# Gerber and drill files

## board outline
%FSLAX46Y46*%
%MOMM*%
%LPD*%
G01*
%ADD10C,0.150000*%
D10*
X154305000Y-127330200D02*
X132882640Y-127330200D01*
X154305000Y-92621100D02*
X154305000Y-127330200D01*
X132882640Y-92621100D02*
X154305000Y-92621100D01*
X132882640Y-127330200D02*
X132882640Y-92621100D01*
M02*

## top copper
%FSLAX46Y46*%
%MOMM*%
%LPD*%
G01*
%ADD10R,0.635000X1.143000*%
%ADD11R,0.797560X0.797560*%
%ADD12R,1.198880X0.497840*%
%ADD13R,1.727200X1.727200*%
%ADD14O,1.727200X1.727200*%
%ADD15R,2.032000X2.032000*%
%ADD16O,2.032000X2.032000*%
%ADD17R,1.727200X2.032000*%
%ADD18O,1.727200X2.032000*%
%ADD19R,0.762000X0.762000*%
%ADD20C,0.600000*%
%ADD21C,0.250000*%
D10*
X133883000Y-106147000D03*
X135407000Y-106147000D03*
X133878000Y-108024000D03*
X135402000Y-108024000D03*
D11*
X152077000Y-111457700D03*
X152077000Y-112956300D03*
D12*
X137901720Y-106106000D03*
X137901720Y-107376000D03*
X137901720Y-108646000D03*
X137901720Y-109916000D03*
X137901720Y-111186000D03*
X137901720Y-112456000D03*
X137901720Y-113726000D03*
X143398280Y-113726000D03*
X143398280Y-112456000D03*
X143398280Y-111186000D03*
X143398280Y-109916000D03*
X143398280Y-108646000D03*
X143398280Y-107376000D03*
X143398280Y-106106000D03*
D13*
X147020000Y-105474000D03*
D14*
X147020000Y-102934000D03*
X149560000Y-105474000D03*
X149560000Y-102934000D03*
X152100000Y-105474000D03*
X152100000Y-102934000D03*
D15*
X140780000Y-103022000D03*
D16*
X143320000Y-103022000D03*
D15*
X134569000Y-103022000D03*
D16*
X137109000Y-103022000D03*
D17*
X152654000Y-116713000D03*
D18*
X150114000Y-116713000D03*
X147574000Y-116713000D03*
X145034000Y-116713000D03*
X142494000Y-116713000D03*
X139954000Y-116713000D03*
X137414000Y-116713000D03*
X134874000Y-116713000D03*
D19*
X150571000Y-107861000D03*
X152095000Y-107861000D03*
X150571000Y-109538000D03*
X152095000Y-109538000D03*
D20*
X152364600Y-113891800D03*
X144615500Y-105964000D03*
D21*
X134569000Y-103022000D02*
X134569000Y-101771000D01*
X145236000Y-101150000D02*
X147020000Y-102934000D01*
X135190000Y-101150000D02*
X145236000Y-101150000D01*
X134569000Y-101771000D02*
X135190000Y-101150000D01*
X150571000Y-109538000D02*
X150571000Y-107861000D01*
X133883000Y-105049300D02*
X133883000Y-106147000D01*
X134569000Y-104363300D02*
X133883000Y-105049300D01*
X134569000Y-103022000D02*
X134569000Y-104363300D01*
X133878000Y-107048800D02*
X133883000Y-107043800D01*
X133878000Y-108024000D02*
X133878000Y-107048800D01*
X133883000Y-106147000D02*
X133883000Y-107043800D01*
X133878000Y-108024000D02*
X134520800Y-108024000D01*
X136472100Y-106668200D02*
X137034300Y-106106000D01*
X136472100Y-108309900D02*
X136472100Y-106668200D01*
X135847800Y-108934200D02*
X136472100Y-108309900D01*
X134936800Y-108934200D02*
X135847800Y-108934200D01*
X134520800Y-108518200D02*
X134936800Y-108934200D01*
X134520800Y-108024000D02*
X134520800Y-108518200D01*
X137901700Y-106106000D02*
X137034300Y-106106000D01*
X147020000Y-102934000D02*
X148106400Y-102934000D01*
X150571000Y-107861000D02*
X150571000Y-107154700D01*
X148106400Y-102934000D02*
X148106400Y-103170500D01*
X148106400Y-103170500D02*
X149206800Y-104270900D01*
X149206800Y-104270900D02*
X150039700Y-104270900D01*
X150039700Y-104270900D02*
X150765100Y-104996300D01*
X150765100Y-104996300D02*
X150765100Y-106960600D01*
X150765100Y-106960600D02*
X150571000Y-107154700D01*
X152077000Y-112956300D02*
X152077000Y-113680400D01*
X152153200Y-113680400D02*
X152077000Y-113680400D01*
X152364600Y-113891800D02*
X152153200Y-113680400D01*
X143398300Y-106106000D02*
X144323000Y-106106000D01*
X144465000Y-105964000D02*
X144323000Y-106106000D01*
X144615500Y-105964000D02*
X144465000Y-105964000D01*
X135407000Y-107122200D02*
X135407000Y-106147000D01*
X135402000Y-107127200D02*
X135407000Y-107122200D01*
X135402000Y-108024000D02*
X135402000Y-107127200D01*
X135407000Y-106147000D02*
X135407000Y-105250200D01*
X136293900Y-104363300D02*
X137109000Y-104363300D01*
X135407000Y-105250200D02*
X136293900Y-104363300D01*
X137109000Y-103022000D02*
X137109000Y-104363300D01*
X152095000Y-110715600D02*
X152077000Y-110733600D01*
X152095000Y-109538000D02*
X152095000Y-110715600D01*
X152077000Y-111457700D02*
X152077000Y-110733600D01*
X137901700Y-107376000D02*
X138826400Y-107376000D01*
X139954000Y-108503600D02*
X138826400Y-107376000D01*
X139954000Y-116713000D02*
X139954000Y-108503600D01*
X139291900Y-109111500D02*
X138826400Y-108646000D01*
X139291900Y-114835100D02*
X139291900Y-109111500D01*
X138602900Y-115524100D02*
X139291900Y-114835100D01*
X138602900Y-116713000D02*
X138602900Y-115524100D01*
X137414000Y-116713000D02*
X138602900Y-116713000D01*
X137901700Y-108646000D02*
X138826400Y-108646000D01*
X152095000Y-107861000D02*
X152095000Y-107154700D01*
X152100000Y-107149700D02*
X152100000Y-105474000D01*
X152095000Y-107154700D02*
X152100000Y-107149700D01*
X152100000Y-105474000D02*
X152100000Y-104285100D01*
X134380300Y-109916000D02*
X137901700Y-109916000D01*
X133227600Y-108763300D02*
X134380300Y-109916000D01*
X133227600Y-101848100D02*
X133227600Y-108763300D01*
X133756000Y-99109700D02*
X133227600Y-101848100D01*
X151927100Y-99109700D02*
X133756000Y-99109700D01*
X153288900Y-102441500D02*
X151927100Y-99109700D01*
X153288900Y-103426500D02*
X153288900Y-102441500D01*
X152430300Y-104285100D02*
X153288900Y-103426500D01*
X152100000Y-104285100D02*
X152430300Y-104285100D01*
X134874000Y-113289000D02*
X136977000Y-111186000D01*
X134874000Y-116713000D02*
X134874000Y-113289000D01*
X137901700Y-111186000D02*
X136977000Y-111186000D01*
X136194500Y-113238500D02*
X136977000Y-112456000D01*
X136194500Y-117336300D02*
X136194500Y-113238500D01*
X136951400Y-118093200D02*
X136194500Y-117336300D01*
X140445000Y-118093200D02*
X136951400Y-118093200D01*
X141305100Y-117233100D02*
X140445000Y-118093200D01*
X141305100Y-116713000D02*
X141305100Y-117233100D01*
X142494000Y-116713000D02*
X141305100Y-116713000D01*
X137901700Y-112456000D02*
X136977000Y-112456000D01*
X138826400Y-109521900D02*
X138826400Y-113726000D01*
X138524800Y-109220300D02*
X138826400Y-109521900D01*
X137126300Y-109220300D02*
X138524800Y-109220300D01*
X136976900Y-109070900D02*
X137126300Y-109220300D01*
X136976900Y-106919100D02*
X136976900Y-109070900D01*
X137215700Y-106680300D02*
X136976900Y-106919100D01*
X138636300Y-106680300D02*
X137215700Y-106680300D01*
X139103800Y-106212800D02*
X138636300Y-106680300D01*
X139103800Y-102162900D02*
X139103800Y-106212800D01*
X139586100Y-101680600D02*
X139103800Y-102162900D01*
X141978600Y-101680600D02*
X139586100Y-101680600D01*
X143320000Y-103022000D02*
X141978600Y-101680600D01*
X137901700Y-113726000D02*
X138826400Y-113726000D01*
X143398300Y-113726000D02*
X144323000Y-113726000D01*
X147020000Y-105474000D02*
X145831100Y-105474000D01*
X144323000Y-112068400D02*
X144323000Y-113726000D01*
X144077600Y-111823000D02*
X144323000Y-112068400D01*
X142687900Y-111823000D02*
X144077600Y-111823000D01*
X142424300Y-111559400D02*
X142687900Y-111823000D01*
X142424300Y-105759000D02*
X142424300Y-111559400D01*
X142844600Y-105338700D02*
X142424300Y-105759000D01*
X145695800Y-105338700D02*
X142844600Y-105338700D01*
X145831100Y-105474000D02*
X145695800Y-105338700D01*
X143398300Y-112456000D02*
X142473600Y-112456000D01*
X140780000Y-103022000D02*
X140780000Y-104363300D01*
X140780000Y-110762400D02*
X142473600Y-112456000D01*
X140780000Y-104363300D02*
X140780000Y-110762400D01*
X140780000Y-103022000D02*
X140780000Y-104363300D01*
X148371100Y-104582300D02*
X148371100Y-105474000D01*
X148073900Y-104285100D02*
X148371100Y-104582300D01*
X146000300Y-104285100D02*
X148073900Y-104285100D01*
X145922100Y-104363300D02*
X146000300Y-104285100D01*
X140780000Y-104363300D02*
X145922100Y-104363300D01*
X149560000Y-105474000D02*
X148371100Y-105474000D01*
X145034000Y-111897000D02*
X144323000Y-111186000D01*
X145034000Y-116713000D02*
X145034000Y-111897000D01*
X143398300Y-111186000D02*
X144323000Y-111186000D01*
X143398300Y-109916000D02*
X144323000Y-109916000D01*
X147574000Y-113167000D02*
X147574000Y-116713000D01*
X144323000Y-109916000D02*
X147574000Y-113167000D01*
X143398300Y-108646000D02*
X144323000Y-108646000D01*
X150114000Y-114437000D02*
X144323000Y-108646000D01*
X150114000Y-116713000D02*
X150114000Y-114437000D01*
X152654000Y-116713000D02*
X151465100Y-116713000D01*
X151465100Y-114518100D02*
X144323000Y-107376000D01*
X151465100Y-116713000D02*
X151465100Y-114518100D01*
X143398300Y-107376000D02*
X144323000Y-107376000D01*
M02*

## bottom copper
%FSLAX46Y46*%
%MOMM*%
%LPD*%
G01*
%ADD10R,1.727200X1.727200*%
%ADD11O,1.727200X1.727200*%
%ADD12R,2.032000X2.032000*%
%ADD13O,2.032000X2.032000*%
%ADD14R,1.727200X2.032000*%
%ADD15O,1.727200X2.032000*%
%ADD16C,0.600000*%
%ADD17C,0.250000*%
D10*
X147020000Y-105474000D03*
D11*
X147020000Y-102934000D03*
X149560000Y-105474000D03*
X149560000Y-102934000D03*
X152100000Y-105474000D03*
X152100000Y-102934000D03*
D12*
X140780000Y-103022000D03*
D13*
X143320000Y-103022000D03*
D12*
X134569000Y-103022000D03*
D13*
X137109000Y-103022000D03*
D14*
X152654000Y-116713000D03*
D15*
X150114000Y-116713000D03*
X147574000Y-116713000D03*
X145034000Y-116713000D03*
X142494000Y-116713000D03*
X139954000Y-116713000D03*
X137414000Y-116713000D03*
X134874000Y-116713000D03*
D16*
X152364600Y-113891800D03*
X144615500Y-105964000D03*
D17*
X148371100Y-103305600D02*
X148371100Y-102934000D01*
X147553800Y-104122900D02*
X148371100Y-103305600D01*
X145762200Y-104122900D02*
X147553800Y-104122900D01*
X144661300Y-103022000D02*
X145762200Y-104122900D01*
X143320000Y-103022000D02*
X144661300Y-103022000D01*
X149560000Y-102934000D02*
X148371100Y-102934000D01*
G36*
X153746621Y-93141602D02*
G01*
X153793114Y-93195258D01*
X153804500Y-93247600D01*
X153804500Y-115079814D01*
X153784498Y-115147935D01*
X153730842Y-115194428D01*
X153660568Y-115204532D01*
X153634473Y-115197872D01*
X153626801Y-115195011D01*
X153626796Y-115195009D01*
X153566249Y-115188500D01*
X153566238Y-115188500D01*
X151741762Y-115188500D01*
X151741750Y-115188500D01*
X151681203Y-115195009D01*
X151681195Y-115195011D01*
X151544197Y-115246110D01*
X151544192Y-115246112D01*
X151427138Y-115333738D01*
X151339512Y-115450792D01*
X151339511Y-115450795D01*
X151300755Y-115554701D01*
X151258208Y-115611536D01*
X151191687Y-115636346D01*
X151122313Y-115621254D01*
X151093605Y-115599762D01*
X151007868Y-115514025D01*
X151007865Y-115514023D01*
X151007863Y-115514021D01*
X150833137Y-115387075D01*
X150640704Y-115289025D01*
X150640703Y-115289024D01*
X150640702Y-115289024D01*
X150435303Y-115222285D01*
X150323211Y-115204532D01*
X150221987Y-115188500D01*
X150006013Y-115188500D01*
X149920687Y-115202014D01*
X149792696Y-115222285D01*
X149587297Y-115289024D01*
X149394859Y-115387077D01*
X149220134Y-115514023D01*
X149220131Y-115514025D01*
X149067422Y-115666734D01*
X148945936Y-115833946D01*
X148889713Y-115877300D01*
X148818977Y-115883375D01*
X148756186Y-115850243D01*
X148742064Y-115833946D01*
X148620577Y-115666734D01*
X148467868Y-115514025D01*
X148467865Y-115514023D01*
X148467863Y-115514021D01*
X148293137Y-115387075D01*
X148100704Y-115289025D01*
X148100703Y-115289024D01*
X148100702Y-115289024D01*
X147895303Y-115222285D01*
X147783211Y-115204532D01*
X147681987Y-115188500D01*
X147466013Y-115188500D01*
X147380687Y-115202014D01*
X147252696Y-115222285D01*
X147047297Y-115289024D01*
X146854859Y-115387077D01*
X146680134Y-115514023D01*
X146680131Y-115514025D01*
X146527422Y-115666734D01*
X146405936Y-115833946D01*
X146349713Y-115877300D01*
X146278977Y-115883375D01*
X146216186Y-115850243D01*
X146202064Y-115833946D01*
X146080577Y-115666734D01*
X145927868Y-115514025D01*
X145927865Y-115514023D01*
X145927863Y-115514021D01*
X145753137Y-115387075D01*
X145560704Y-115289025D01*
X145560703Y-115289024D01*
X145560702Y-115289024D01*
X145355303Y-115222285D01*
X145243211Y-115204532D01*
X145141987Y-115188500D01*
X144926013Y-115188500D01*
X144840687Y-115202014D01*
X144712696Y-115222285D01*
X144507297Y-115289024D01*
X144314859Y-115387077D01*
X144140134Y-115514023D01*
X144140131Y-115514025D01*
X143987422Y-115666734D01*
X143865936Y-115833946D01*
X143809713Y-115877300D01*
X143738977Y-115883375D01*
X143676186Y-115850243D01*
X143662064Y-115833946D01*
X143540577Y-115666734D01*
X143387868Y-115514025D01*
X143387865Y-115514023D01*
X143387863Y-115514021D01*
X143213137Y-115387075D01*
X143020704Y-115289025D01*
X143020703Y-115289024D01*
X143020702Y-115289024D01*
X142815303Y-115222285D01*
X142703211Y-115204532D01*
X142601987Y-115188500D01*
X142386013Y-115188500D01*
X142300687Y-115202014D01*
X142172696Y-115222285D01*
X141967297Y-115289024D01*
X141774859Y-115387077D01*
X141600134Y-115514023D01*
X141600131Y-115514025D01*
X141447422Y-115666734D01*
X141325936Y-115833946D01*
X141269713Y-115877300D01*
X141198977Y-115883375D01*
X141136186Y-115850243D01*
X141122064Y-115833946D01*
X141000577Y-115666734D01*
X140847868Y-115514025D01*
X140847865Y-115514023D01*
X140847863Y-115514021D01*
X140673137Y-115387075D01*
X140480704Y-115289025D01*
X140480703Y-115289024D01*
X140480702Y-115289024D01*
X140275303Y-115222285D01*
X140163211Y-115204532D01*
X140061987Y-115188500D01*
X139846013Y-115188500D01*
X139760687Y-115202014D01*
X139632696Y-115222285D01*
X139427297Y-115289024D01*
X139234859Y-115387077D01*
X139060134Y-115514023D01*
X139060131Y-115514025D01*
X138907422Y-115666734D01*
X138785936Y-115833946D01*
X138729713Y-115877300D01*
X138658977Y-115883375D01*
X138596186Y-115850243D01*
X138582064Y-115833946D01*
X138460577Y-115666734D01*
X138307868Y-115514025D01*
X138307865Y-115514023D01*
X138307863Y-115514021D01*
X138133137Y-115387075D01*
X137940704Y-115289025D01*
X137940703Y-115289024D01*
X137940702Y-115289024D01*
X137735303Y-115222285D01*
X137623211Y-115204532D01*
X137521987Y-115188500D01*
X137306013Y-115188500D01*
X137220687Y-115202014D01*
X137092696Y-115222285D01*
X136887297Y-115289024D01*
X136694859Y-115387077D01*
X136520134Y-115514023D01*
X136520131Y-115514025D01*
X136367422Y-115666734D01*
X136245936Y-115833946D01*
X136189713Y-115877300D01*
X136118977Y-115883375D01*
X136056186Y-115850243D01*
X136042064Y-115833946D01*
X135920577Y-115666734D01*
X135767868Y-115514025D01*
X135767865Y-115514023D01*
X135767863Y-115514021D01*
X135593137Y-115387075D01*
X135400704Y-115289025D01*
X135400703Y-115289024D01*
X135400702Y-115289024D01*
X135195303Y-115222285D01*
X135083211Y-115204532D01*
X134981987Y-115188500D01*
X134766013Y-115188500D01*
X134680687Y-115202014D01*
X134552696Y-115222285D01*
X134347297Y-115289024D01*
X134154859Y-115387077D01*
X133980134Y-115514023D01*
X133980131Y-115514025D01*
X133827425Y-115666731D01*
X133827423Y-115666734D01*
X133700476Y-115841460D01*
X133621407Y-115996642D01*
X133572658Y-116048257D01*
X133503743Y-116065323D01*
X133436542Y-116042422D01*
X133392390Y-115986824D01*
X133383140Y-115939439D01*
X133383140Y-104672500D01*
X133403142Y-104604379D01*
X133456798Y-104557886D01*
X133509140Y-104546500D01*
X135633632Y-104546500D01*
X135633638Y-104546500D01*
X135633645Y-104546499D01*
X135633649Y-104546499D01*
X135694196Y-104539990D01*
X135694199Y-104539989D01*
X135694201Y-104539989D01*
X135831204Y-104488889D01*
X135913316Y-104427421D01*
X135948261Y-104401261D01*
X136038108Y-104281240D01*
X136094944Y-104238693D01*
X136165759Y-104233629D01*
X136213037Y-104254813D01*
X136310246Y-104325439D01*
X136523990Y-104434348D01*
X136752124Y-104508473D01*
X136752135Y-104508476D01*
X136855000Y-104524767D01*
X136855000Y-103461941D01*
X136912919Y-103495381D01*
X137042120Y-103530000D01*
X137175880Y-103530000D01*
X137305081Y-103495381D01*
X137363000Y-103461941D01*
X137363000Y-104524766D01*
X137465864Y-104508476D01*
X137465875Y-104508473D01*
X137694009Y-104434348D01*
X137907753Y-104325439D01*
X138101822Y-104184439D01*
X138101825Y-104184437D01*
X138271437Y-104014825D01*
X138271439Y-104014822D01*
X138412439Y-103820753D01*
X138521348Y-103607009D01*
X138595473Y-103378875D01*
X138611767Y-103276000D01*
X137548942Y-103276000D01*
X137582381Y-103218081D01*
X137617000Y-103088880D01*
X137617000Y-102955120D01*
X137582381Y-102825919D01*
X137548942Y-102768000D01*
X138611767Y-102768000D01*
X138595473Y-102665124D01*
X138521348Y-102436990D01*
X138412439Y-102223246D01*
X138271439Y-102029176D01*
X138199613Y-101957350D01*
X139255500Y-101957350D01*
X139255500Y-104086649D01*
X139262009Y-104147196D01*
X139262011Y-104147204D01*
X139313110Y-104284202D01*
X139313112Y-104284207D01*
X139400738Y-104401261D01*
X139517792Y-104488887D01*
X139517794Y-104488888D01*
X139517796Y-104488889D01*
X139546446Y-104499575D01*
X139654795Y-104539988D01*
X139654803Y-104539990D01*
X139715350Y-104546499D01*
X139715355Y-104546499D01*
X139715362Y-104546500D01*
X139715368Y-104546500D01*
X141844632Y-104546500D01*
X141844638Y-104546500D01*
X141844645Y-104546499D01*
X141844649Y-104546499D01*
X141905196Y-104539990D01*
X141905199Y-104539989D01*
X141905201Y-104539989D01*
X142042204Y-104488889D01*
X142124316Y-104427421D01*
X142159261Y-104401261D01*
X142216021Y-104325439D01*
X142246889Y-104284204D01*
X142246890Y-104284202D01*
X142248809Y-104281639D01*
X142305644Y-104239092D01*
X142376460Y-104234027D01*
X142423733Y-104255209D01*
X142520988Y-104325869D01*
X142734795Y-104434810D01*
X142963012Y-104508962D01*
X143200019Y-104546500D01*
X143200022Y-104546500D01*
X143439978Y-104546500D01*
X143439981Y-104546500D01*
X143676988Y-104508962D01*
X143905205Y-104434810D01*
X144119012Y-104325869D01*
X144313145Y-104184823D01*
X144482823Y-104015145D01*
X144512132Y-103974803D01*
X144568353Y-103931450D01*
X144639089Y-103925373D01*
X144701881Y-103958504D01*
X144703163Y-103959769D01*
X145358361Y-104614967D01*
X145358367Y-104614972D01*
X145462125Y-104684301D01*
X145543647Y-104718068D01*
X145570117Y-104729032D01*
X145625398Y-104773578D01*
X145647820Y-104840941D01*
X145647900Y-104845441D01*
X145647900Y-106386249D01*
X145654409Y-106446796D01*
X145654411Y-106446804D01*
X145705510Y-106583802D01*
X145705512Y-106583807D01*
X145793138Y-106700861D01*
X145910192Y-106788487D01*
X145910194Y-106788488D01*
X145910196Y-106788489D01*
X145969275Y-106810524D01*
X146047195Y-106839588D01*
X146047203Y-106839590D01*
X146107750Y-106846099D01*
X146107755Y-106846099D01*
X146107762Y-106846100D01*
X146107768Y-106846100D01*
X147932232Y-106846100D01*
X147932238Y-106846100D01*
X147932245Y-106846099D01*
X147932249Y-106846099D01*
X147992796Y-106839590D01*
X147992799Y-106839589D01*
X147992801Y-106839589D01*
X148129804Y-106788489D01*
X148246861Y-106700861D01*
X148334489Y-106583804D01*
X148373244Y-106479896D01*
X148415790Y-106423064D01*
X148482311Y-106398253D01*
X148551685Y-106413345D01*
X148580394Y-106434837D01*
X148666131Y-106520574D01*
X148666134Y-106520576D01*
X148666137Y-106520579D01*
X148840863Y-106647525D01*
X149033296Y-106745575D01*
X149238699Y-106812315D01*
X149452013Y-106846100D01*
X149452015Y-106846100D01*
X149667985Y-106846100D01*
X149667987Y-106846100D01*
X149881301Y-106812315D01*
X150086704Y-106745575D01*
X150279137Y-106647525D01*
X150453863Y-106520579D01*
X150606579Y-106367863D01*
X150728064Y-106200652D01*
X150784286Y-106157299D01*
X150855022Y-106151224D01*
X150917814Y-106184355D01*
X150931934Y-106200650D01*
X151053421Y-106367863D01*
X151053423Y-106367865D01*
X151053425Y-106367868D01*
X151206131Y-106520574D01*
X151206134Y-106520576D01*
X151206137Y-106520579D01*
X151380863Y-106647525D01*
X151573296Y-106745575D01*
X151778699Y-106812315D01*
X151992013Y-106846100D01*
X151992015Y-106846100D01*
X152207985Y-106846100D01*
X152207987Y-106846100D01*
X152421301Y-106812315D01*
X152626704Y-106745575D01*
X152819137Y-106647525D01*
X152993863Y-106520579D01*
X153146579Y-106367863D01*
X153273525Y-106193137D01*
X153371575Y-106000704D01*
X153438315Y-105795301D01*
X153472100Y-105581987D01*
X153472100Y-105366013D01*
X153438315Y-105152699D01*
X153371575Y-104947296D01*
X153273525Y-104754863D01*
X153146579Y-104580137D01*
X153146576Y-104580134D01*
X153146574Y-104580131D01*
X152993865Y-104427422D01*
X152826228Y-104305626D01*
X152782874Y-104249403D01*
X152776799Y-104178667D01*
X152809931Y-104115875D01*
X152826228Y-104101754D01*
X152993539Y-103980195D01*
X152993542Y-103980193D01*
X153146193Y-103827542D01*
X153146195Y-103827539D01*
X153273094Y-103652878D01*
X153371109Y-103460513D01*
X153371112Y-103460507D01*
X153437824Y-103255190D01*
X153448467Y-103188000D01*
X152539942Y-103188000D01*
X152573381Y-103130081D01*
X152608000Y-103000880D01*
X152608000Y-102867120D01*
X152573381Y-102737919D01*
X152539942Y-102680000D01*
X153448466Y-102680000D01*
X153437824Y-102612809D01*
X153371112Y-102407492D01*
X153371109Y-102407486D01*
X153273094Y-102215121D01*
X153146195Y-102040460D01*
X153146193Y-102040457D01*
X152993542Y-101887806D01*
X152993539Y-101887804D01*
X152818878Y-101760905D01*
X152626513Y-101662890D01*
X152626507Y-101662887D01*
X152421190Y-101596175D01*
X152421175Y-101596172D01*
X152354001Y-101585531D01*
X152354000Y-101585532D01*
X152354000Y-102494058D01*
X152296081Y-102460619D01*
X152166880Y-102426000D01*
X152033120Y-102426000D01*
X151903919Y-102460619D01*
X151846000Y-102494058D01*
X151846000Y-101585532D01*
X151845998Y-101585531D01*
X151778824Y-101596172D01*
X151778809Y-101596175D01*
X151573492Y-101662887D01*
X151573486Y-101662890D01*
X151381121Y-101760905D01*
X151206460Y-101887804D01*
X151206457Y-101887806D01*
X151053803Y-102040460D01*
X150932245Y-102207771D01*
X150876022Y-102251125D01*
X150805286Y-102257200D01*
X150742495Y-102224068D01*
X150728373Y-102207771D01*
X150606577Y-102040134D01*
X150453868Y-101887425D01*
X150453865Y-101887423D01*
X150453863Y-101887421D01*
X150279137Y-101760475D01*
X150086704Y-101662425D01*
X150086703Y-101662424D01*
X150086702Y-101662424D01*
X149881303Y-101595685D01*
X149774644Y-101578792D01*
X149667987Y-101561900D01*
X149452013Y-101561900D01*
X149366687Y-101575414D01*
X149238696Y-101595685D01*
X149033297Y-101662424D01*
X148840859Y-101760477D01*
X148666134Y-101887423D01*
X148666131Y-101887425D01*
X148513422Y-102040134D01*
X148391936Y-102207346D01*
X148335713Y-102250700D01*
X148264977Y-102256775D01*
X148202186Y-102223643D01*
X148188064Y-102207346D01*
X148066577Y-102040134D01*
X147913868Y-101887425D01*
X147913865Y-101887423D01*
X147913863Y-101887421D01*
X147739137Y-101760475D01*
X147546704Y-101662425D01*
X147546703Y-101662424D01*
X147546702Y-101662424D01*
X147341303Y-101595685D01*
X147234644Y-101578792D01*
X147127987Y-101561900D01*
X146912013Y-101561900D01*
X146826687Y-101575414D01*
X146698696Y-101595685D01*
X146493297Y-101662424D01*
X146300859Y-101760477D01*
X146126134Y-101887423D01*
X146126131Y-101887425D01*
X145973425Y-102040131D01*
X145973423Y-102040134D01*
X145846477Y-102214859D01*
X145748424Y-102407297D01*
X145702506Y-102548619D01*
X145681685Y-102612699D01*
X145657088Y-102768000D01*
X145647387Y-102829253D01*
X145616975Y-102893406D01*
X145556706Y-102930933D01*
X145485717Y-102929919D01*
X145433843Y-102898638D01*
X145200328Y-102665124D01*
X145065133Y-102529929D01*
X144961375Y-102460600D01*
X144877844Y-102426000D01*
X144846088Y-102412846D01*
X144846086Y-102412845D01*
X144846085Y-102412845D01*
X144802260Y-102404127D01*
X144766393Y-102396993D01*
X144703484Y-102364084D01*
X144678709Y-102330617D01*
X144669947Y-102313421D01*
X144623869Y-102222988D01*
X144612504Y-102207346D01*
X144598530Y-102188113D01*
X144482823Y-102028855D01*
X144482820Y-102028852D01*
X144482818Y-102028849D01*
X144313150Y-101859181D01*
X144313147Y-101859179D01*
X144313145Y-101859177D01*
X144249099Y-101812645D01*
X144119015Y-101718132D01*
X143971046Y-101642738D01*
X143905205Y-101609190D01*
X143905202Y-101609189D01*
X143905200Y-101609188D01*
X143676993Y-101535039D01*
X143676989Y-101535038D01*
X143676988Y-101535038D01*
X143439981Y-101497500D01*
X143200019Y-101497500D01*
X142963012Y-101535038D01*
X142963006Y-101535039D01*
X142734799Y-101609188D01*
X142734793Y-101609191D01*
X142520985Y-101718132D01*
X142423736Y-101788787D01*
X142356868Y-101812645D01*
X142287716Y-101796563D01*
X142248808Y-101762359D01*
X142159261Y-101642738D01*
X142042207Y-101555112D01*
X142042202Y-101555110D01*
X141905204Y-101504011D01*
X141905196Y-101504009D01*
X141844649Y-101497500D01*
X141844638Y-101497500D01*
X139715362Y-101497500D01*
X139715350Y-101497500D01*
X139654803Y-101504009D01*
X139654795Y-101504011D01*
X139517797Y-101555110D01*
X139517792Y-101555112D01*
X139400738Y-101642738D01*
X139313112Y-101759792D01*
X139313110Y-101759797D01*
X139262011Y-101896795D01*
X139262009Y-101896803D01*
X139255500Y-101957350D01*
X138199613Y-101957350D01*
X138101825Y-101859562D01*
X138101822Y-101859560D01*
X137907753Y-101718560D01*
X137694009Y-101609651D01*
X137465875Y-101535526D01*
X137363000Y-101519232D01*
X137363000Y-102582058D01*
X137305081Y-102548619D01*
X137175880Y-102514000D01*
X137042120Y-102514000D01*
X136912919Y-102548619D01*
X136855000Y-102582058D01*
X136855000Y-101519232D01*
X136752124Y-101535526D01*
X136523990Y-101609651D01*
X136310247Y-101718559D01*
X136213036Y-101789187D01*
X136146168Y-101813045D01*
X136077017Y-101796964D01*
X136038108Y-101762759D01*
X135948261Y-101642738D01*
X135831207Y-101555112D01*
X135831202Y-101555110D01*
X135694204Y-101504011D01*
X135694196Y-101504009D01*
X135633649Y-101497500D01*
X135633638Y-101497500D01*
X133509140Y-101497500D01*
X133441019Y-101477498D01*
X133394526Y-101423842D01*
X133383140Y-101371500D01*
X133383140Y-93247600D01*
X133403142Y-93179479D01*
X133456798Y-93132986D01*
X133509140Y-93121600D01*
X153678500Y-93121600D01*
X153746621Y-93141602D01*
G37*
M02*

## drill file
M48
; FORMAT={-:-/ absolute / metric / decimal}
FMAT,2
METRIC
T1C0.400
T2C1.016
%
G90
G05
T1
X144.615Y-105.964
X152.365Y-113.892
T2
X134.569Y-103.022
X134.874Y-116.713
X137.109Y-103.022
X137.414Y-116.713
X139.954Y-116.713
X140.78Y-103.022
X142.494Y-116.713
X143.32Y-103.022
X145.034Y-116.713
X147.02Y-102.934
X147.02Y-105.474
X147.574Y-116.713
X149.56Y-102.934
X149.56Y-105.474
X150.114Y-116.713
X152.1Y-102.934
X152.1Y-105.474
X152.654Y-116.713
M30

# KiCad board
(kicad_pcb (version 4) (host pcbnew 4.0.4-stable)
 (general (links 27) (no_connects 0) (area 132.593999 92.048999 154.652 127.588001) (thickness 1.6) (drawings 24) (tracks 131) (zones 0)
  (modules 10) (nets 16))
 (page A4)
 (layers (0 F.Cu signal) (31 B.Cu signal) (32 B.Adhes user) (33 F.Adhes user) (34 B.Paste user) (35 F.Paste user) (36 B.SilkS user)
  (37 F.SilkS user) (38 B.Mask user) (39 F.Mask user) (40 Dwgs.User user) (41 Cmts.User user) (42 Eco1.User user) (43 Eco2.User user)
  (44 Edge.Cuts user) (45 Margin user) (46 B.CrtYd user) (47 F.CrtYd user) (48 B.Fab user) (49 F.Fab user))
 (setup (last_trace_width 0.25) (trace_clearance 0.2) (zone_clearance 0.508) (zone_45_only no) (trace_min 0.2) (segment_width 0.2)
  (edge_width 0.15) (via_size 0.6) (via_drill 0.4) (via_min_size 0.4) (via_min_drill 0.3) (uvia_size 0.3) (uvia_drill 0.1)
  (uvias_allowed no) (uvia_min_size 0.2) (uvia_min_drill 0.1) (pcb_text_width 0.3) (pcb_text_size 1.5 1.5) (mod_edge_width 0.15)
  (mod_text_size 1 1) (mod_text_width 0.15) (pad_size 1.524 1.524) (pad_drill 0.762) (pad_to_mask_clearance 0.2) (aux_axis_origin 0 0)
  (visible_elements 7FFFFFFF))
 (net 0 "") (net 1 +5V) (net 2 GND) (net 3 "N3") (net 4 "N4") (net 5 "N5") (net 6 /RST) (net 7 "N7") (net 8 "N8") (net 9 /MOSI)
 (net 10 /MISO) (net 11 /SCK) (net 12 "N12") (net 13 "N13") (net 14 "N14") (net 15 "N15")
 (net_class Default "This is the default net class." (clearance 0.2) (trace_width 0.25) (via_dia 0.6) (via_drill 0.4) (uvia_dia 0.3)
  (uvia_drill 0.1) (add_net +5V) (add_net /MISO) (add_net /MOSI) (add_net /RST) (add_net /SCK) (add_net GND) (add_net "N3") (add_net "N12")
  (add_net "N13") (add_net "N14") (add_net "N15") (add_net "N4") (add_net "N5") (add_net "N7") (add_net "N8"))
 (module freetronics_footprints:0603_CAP (layer F.Cu) (at 134.645 106.147)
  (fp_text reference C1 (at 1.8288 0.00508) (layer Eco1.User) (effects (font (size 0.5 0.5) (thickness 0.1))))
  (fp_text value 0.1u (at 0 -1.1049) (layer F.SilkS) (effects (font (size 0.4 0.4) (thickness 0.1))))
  (pad 1 smd rect (at -0.762 0) (size 0.635 1.143) (layers F.Cu F.Paste F.Mask) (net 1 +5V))
  (pad 2 smd rect (at 0.762 0) (size 0.635 1.143) (layers F.Cu F.Paste F.Mask) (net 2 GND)))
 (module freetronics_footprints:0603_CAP (layer F.Cu) (at 134.64 108.024)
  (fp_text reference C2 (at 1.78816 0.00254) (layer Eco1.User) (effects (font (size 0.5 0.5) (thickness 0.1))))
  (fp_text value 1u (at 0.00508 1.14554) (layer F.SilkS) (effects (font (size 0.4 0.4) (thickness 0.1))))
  (pad 1 smd rect (at -0.762 0) (size 0.635 1.143) (layers F.Cu F.Paste F.Mask) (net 1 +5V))
  (pad 2 smd rect (at 0.762 0) (size 0.635 1.143) (layers F.Cu F.Paste F.Mask) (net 2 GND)))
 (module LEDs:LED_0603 (layer F.Cu) (at 152.077 112.207 90)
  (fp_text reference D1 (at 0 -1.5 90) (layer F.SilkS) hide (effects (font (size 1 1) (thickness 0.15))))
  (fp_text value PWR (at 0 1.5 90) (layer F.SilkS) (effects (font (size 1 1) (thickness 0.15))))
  (pad 2 smd rect (at 0.7493 0 270) (size 0.79756 0.79756) (layers F.Cu F.Paste F.Mask) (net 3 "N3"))
  (pad 1 smd rect (at -0.7493 0 270) (size 0.79756 0.79756) (layers F.Cu F.Paste F.Mask) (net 2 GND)))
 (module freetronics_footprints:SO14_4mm (layer F.Cu) (at 140.65 109.916 270)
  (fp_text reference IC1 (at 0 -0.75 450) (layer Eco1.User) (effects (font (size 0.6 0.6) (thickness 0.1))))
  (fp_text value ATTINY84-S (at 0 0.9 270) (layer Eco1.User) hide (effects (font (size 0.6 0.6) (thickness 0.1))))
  (pad 1 smd rect (at -3.81 2.74828 90) (size 0.49784 1.19888) (layers F.Cu F.Paste F.Mask) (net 1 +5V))
  (pad 2 smd rect (at -2.54 2.74828 90) (size 0.49784 1.19888) (layers F.Cu F.Paste F.Mask) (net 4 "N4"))
  (pad 3 smd rect (at -1.27 2.74828 90) (size 0.49784 1.19888) (layers F.Cu F.Paste F.Mask) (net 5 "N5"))
  (pad 4 smd rect (at 0 2.74828 90) (size 0.49784 1.19888) (layers F.Cu F.Paste F.Mask) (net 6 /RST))
  (pad 5 smd rect (at 1.27 2.74828 90) (size 0.49784 1.19888) (layers F.Cu F.Paste F.Mask) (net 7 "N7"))
  (pad 6 smd rect (at 2.54 2.74828 90) (size 0.49784 1.19888) (layers F.Cu F.Paste F.Mask) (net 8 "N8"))
  (pad 7 smd rect (at 3.81 2.74828 90) (size 0.49784 1.19888) (layers F.Cu F.Paste F.Mask) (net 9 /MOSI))
  (pad 8 smd rect (at 3.81 -2.74828 270) (size 0.49784 1.19888) (layers F.Cu F.Paste F.Mask) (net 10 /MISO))
  (pad 9 smd rect (at 2.54 -2.74828 270) (size 0.49784 1.19888) (layers F.Cu F.Paste F.Mask) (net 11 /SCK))
  (pad 10 smd rect (at 1.27 -2.74828 270) (size 0.49784 1.19888) (layers F.Cu F.Paste F.Mask) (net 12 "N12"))
  (pad 11 smd rect (at 0 -2.74828 270) (size 0.49784 1.19888) (layers F.Cu F.Paste F.Mask) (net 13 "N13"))
  (pad 12 smd rect (at -1.27 -2.74828 270) (size 0.49784 1.19888) (layers F.Cu F.Paste F.Mask) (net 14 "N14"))
  (pad 13 smd rect (at -2.54 -2.74828 270) (size 0.49784 1.19888) (layers F.Cu F.Paste F.Mask) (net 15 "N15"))
  (pad 14 smd rect (at -3.81 -2.74828 270) (size 0.49784 1.19888) (layers F.Cu F.Paste F.Mask) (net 2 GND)))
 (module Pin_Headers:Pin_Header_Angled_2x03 (layer F.Cu) (at 147.02 105.474 90)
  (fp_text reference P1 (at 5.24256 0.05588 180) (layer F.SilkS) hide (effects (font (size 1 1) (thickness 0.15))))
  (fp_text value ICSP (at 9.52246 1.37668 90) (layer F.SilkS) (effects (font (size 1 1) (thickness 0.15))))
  (pad 1 thru_hole rect (at 0 0 90) (size 1.7272 1.7272) (drill 1.016) (layers *.Cu *.Mask F.SilkS) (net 10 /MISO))
  (pad 2 thru_hole oval (at 2.54 0 90) (size 1.7272 1.7272) (drill 1.016) (layers *.Cu *.Mask F.SilkS) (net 1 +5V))
  (pad 3 thru_hole oval (at 0 2.54 90) (size 1.7272 1.7272) (drill 1.016) (layers *.Cu *.Mask F.SilkS) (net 11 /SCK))
  (pad 4 thru_hole oval (at 2.54 2.54 90) (size 1.7272 1.7272) (drill 1.016) (layers *.Cu *.Mask F.SilkS) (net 9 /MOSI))
  (pad 5 thru_hole oval (at 0 5.08 90) (size 1.7272 1.7272) (drill 1.016) (layers *.Cu *.Mask F.SilkS) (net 6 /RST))
  (pad 6 thru_hole oval (at 2.54 5.08 90) (size 1.7272 1.7272) (drill 1.016) (layers *.Cu *.Mask F.SilkS) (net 2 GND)))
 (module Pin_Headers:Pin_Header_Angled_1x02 (layer F.Cu) (at 140.78 103.022 90)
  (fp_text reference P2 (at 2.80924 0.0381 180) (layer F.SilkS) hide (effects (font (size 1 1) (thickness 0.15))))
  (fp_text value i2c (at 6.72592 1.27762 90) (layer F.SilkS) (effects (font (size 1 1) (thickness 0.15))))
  (pad 1 thru_hole rect (at 0 0 90) (size 2.032 2.032) (drill 1.016) (layers *.Cu *.Mask F.SilkS) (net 11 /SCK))
  (pad 2 thru_hole oval (at 0 2.54 90) (size 2.032 2.032) (drill 1.016) (layers *.Cu *.Mask F.SilkS) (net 9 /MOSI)))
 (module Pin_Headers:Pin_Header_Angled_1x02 (layer F.Cu) (at 134.569 103.022 90)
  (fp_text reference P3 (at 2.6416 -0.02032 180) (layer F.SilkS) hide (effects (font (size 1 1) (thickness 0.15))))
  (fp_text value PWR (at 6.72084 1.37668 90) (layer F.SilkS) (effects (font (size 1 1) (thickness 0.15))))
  (pad 1 thru_hole rect (at 0 0 90) (size 2.032 2.032) (drill 1.016) (layers *.Cu *.Mask F.SilkS) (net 1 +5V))
  (pad 2 thru_hole oval (at 0 2.54 90) (size 2.032 2.032) (drill 1.016) (layers *.Cu *.Mask F.SilkS) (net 2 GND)))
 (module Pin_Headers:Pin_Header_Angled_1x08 (layer F.Cu) (at 152.654 116.713 270)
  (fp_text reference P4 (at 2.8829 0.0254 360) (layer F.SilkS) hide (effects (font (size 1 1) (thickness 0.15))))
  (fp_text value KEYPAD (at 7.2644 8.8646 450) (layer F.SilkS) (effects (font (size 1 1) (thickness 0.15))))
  (pad 1 thru_hole rect (at 0 0 270) (size 2.032 1.7272) (drill 1.016) (layers *.Cu *.Mask F.SilkS) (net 15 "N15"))
  (pad 2 thru_hole oval (at 0 2.54 270) (size 2.032 1.7272) (drill 1.016) (layers *.Cu *.Mask F.SilkS) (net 14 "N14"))
  (pad 3 thru_hole oval (at 0 5.08 270) (size 2.032 1.7272) (drill 1.016) (layers *.Cu *.Mask F.SilkS) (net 13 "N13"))
  (pad 4 thru_hole oval (at 0 7.62 270) (size 2.032 1.7272) (drill 1.016) (layers *.Cu *.Mask F.SilkS) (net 12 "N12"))
  (pad 5 thru_hole oval (at 0 10.16 270) (size 2.032 1.7272) (drill 1.016) (layers *.Cu *.Mask F.SilkS) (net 8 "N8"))
  (pad 6 thru_hole oval (at 0 12.7 270) (size 2.032 1.7272) (drill 1.016) (layers *.Cu *.Mask F.SilkS) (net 4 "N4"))
  (pad 7 thru_hole oval (at 0 15.24 270) (size 2.032 1.7272) (drill 1.016) (layers *.Cu *.Mask F.SilkS) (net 5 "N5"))
  (pad 8 thru_hole oval (at 0 17.78 270) (size 2.032 1.7272) (drill 1.016) (layers *.Cu *.Mask F.SilkS) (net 7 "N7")))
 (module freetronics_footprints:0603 (layer F.Cu) (at 151.333 107.861)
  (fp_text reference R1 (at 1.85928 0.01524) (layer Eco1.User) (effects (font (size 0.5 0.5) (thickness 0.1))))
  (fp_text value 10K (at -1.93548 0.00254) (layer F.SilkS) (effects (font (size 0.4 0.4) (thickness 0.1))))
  (pad 1 smd rect (at -0.762 0) (size 0.762 0.762) (layers F.Cu F.Paste F.Mask) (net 1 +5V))
  (pad 2 smd rect (at 0.762 0) (size 0.762 0.762) (layers F.Cu F.Paste F.Mask) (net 6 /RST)))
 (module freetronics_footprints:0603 (layer F.Cu) (at 151.333 109.538)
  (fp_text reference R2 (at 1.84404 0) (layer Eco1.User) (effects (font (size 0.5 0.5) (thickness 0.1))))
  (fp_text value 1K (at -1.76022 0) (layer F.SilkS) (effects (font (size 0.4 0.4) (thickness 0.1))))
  (pad 1 smd rect (at -0.762 0) (size 0.762 0.762) (layers F.Cu F.Paste F.Mask) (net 1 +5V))
  (pad 2 smd rect (at 0.762 0) (size 0.762 0.762) (layers F.Cu F.Paste F.Mask) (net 3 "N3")))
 (gr_line (start 154.305 127.3302) (end 132.88264 127.3302) (angle 90) (layer Edge.Cuts) (width 0.15))
 (gr_line (start 154.305 92.6211) (end 154.305 127.3302) (angle 90) (layer Edge.Cuts) (width 0.15))
 (gr_line (start 132.88264 92.6211) (end 154.305 92.6211) (angle 90) (layer Edge.Cuts) (width 0.15))
 (gr_line (start 132.88264 127.3302) (end 132.88264 92.6211) (angle 90) (layer Edge.Cuts) (width 0.15))
 (segment (start 134.569 103.022) (end 134.569 101.771) (width 0.25) (layer F.Cu) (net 1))
 (segment (start 145.236 101.15) (end 147.02 102.934) (width 0.25) (layer F.Cu) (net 1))
 (segment (start 135.19 101.15) (end 145.236 101.15) (width 0.25) (layer F.Cu) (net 1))
 (segment (start 134.569 101.771) (end 135.19 101.15) (width 0.25) (layer F.Cu) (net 1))
 (segment (start 150.571 109.538) (end 150.571 107.861) (width 0.25) (layer F.Cu) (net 1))
 (segment (start 133.883 105.0493) (end 133.883 106.147) (width 0.25) (layer F.Cu) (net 1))
 (segment (start 134.569 104.3633) (end 133.883 105.0493) (width 0.25) (layer F.Cu) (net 1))
 (segment (start 134.569 103.022) (end 134.569 104.3633) (width 0.25) (layer F.Cu) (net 1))
 (segment (start 133.878 107.0488) (end 133.883 107.0438) (width 0.25) (layer F.Cu) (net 1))
 (segment (start 133.878 108.024) (end 133.878 107.0488) (width 0.25) (layer F.Cu) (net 1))
 (segment (start 133.883 106.147) (end 133.883 107.0438) (width 0.25) (layer F.Cu) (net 1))
 (segment (start 133.878 108.024) (end 134.5208 108.024) (width 0.25) (layer F.Cu) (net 1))
 (segment (start 136.4721 106.6682) (end 137.0343 106.106) (width 0.25) (layer F.Cu) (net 1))
 (segment (start 136.4721 108.3099) (end 136.4721 106.6682) (width 0.25) (layer F.Cu) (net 1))
 (segment (start 135.8478 108.9342) (end 136.4721 108.3099) (width 0.25) (layer F.Cu) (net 1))
 (segment (start 134.9368 108.9342) (end 135.8478 108.9342) (width 0.25) (layer F.Cu) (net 1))
 (segment (start 134.5208 108.5182) (end 134.9368 108.9342) (width 0.25) (layer F.Cu) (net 1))
 (segment (start 134.5208 108.024) (end 134.5208 108.5182) (width 0.25) (layer F.Cu) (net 1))
 (segment (start 137.9017 106.106) (end 137.0343 106.106) (width 0.25) (layer F.Cu) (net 1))
 (segment (start 147.02 102.934) (end 148.1064 102.934) (width 0.25) (layer F.Cu) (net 1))
 (segment (start 150.571 107.861) (end 150.571 107.1547) (width 0.25) (layer F.Cu) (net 1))
 (segment (start 148.1064 102.934) (end 148.1064 103.1705) (width 0.25) (layer F.Cu) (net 1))
 (segment (start 148.1064 103.1705) (end 149.2068 104.2709) (width 0.25) (layer F.Cu) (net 1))
 (segment (start 149.2068 104.2709) (end 150.0397 104.2709) (width 0.25) (layer F.Cu) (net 1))
 (segment (start 150.0397 104.2709) (end 150.7651 104.9963) (width 0.25) (layer F.Cu) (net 1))
 (segment (start 150.7651 104.9963) (end 150.7651 106.9606) (width 0.25) (layer F.Cu) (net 1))
 (segment (start 150.7651 106.9606) (end 150.571 107.1547) (width 0.25) (layer F.Cu) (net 1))
 (via (at 152.3646 113.8918) (size 0.6) (layers F.Cu B.Cu) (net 2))
 (via (at 144.6155 105.964) (size 0.6) (layers F.Cu B.Cu) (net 2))
 (segment (start 152.077 112.9563) (end 152.077 113.6804) (width 0.25) (layer F.Cu) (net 2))
 (segment (start 152.1532 113.6804) (end 152.077 113.6804) (width 0.25) (layer F.Cu) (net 2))
 (segment (start 152.3646 113.8918) (end 152.1532 113.6804) (width 0.25) (layer F.Cu) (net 2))
 (segment (start 143.3983 106.106) (end 144.323 106.106) (width 0.25) (layer F.Cu) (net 2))
 (segment (start 144.465 105.964) (end 144.323 106.106) (width 0.25) (layer F.Cu) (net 2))
 (segment (start 144.6155 105.964) (end 144.465 105.964) (width 0.25) (layer F.Cu) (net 2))
 (segment (start 135.407 107.1222) (end 135.407 106.147) (width 0.25) (layer F.Cu) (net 2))
 (segment (start 135.402 107.1272) (end 135.407 107.1222) (width 0.25) (layer F.Cu) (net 2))
 (segment (start 135.402 108.024) (end 135.402 107.1272) (width 0.25) (layer F.Cu) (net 2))
 (segment (start 135.407 106.147) (end 135.407 105.2502) (width 0.25) (layer F.Cu) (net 2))
 (segment (start 136.2939 104.3633) (end 137.109 104.3633) (width 0.25) (layer F.Cu) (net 2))
 (segment (start 135.407 105.2502) (end 136.2939 104.3633) (width 0.25) (layer F.Cu) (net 2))
 (segment (start 137.109 103.022) (end 137.109 104.3633) (width 0.25) (layer F.Cu) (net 2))
 (segment (start 152.095 110.7156) (end 152.077 110.7336) (width 0.25) (layer F.Cu) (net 3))
 (segment (start 152.095 109.538) (end 152.095 110.7156) (width 0.25) (layer F.Cu) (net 3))
 (segment (start 152.077 111.4577) (end 152.077 110.7336) (width 0.25) (layer F.Cu) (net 3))
 (segment (start 137.9017 107.376) (end 138.8264 107.376) (width 0.25) (layer F.Cu) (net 4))
 (segment (start 139.954 108.5036) (end 138.8264 107.376) (width 0.25) (layer F.Cu) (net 4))
 (segment (start 139.954 116.713) (end 139.954 108.5036) (width 0.25) (layer F.Cu) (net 4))
 (segment (start 139.2919 109.1115) (end 138.8264 108.646) (width 0.25) (layer F.Cu) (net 5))
 (segment (start 139.2919 114.8351) (end 139.2919 109.1115) (width 0.25) (layer F.Cu) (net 5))
 (segment (start 138.6029 115.5241) (end 139.2919 114.8351) (width 0.25) (layer F.Cu) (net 5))
 (segment (start 138.6029 116.713) (end 138.6029 115.5241) (width 0.25) (layer F.Cu) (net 5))
 (segment (start 137.414 116.713) (end 138.6029 116.713) (width 0.25) (layer F.Cu) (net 5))
 (segment (start 137.9017 108.646) (end 138.8264 108.646) (width 0.25) (layer F.Cu) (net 5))
 (segment (start 152.095 107.861) (end 152.095 107.1547) (width 0.25) (layer F.Cu) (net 6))
 (segment (start 152.1 107.1497) (end 152.1 105.474) (width 0.25) (layer F.Cu) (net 6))
 (segment (start 152.095 107.1547) (end 152.1 107.1497) (width 0.25) (layer F.Cu) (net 6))
 (segment (start 152.1 105.474) (end 152.1 104.2851) (width 0.25) (layer F.Cu) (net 6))
 (segment (start 134.3803 109.916) (end 137.9017 109.916) (width 0.25) (layer F.Cu) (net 6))
 (segment (start 133.2276 108.7633) (end 134.3803 109.916) (width 0.25) (layer F.Cu) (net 6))
 (segment (start 133.2276 101.8481) (end 133.2276 108.7633) (width 0.25) (layer F.Cu) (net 6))
 (segment (start 133.756 99.1097) (end 133.2276 101.8481) (width 0.25) (layer F.Cu) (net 6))
 (segment (start 151.9271 99.1097) (end 133.756 99.1097) (width 0.25) (layer F.Cu) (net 6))
 (segment (start 153.2889 102.4415) (end 151.9271 99.1097) (width 0.25) (layer F.Cu) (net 6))
 (segment (start 153.2889 103.4265) (end 153.2889 102.4415) (width 0.25) (layer F.Cu) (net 6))
 (segment (start 152.4303 104.2851) (end 153.2889 103.4265) (width 0.25) (layer F.Cu) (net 6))
 (segment (start 152.1 104.2851) (end 152.4303 104.2851) (width 0.25) (layer F.Cu) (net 6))
 (segment (start 134.874 113.289) (end 136.977 111.186) (width 0.25) (layer F.Cu) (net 7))
 (segment (start 134.874 116.713) (end 134.874 113.289) (width 0.25) (layer F.Cu) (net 7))
 (segment (start 137.9017 111.186) (end 136.977 111.186) (width 0.25) (layer F.Cu) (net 7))
 (segment (start 136.1945 113.2385) (end 136.977 112.456) (width 0.25) (layer F.Cu) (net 8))
 (segment (start 136.1945 117.3363) (end 136.1945 113.2385) (width 0.25) (layer F.Cu) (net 8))
 (segment (start 136.9514 118.0932) (end 136.1945 117.3363) (width 0.25) (layer F.Cu) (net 8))
 (segment (start 140.445 118.0932) (end 136.9514 118.0932) (width 0.25) (layer F.Cu) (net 8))
 (segment (start 141.3051 117.2331) (end 140.445 118.0932) (width 0.25) (layer F.Cu) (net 8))
 (segment (start 141.3051 116.713) (end 141.3051 117.2331) (width 0.25) (layer F.Cu) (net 8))
 (segment (start 142.494 116.713) (end 141.3051 116.713) (width 0.25) (layer F.Cu) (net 8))
 (segment (start 137.9017 112.456) (end 136.977 112.456) (width 0.25) (layer F.Cu) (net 8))
 (segment (start 148.3711 103.3056) (end 148.3711 102.934) (width 0.25) (layer B.Cu) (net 9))
 (segment (start 147.5538 104.1229) (end 148.3711 103.3056) (width 0.25) (layer B.Cu) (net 9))
 (segment (start 145.7622 104.1229) (end 147.5538 104.1229) (width 0.25) (layer B.Cu) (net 9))
 (segment (start 144.6613 103.022) (end 145.7622 104.1229) (width 0.25) (layer B.Cu) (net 9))
 (segment (start 143.32 103.022) (end 144.6613 103.022) (width 0.25) (layer B.Cu) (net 9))
 (segment (start 149.56 102.934) (end 148.3711 102.934) (width 0.25) (layer B.Cu) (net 9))
 (segment (start 138.8264 109.5219) (end 138.8264 113.726) (width 0.25) (layer F.Cu) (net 9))
 (segment (start 138.5248 109.2203) (end 138.8264 109.5219) (width 0.25) (layer F.Cu) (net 9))
 (segment (start 137.1263 109.2203) (end 138.5248 109.2203) (width 0.25) (layer F.Cu) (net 9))
 (segment (start 136.9769 109.0709) (end 137.1263 109.2203) (width 0.25) (layer F.Cu) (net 9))
 (segment (start 136.9769 106.9191) (end 136.9769 109.0709) (width 0.25) (layer F.Cu) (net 9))
 (segment (start 137.2157 106.6803) (end 136.9769 106.9191) (width 0.25) (layer F.Cu) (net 9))
 (segment (start 138.6363 106.6803) (end 137.2157 106.6803) (width 0.25) (layer F.Cu) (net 9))
 (segment (start 139.1038 106.2128) (end 138.6363 106.6803) (width 0.25) (layer F.Cu) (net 9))
 (segment (start 139.1038 102.1629) (end 139.1038 106.2128) (width 0.25) (layer F.Cu) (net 9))
 (segment (start 139.5861 101.6806) (end 139.1038 102.1629) (width 0.25) (layer F.Cu) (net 9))
 (segment (start 141.9786 101.6806) (end 139.5861 101.6806) (width 0.25) (layer F.Cu) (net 9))
 (segment (start 143.32 103.022) (end 141.9786 101.6806) (width 0.25) (layer F.Cu) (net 9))
 (segment (start 137.9017 113.726) (end 138.8264 113.726) (width 0.25) (layer F.Cu) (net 9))
 (segment (start 143.3983 113.726) (end 144.323 113.726) (width 0.25) (layer F.Cu) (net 10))
 (segment (start 147.02 105.474) (end 145.8311 105.474) (width 0.25) (layer F.Cu) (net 10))
 (segment (start 144.323 112.0684) (end 144.323 113.726) (width 0.25) (layer F.Cu) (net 10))
 (segment (start 144.0776 111.823) (end 144.323 112.0684) (width 0.25) (layer F.Cu) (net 10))
 (segment (start 142.6879 111.823) (end 144.0776 111.823) (width 0.25) (layer F.Cu) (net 10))
 (segment (start 142.4243 111.5594) (end 142.6879 111.823) (width 0.25) (layer F.Cu) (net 10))
 (segment (start 142.4243 105.759) (end 142.4243 111.5594) (width 0.25) (layer F.Cu) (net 10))
 (segment (start 142.8446 105.3387) (end 142.4243 105.759) (width 0.25) (layer F.Cu) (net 10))
 (segment (start 145.6958 105.3387) (end 142.8446 105.3387) (width 0.25) (layer F.Cu) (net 10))
 (segment (start 145.8311 105.474) (end 145.6958 105.3387) (width 0.25) (layer F.Cu) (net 10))
 (segment (start 143.3983 112.456) (end 142.4736 112.456) (width 0.25) (layer F.Cu) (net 11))
 (segment (start 140.78 103.022) (end 140.78 104.3633) (width 0.25) (layer F.Cu) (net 11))
 (segment (start 140.78 110.7624) (end 142.4736 112.456) (width 0.25) (layer F.Cu) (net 11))
 (segment (start 140.78 104.3633) (end 140.78 110.7624) (width 0.25) (layer F.Cu) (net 11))
 (segment (start 140.78 103.022) (end 140.78 104.3633) (width 0.25) (layer F.Cu) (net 11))
 (segment (start 148.3711 104.5823) (end 148.3711 105.474) (width 0.25) (layer F.Cu) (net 11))
 (segment (start 148.0739 104.2851) (end 148.3711 104.5823) (width 0.25) (layer F.Cu) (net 11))
 (segment (start 146.0003 104.2851) (end 148.0739 104.2851) (width 0.25) (layer F.Cu) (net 11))
 (segment (start 145.9221 104.3633) (end 146.0003 104.2851) (width 0.25) (layer F.Cu) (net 11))
 (segment (start 140.78 104.3633) (end 145.9221 104.3633) (width 0.25) (layer F.Cu) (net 11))
 (segment (start 149.56 105.474) (end 148.3711 105.474) (width 0.25) (layer F.Cu) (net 11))
 (segment (start 145.034 111.897) (end 144.323 111.186) (width 0.25) (layer F.Cu) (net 12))
 (segment (start 145.034 116.713) (end 145.034 111.897) (width 0.25) (layer F.Cu) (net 12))
 (segment (start 143.3983 111.186) (end 144.323 111.186) (width 0.25) (layer F.Cu) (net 12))
 (segment (start 143.3983 109.916) (end 144.323 109.916) (width 0.25) (layer F.Cu) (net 13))
 (segment (start 147.574 113.167) (end 147.574 116.713) (width 0.25) (layer F.Cu) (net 13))
 (segment (start 144.323 109.916) (end 147.574 113.167) (width 0.25) (layer F.Cu) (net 13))
 (segment (start 143.3983 108.646) (end 144.323 108.646) (width 0.25) (layer F.Cu) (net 14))
 (segment (start 150.114 114.437) (end 144.323 108.646) (width 0.25) (layer F.Cu) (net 14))
 (segment (start 150.114 116.713) (end 150.114 114.437) (width 0.25) (layer F.Cu) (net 14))
 (segment (start 152.654 116.713) (end 151.4651 116.713) (width 0.25) (layer F.Cu) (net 15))
 (segment (start 151.4651 114.5181) (end 144.323 107.376) (width 0.25) (layer F.Cu) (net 15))
 (segment (start 151.4651 116.713) (end 151.4651 114.5181) (width 0.25) (layer F.Cu) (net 15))
 (segment (start 143.3983 107.376) (end 144.323 107.376) (width 0.25) (layer F.Cu) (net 15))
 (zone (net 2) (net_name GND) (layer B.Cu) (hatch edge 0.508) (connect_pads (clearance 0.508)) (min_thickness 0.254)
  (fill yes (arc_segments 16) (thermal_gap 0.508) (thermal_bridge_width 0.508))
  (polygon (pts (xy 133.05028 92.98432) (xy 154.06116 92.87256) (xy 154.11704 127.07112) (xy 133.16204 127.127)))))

